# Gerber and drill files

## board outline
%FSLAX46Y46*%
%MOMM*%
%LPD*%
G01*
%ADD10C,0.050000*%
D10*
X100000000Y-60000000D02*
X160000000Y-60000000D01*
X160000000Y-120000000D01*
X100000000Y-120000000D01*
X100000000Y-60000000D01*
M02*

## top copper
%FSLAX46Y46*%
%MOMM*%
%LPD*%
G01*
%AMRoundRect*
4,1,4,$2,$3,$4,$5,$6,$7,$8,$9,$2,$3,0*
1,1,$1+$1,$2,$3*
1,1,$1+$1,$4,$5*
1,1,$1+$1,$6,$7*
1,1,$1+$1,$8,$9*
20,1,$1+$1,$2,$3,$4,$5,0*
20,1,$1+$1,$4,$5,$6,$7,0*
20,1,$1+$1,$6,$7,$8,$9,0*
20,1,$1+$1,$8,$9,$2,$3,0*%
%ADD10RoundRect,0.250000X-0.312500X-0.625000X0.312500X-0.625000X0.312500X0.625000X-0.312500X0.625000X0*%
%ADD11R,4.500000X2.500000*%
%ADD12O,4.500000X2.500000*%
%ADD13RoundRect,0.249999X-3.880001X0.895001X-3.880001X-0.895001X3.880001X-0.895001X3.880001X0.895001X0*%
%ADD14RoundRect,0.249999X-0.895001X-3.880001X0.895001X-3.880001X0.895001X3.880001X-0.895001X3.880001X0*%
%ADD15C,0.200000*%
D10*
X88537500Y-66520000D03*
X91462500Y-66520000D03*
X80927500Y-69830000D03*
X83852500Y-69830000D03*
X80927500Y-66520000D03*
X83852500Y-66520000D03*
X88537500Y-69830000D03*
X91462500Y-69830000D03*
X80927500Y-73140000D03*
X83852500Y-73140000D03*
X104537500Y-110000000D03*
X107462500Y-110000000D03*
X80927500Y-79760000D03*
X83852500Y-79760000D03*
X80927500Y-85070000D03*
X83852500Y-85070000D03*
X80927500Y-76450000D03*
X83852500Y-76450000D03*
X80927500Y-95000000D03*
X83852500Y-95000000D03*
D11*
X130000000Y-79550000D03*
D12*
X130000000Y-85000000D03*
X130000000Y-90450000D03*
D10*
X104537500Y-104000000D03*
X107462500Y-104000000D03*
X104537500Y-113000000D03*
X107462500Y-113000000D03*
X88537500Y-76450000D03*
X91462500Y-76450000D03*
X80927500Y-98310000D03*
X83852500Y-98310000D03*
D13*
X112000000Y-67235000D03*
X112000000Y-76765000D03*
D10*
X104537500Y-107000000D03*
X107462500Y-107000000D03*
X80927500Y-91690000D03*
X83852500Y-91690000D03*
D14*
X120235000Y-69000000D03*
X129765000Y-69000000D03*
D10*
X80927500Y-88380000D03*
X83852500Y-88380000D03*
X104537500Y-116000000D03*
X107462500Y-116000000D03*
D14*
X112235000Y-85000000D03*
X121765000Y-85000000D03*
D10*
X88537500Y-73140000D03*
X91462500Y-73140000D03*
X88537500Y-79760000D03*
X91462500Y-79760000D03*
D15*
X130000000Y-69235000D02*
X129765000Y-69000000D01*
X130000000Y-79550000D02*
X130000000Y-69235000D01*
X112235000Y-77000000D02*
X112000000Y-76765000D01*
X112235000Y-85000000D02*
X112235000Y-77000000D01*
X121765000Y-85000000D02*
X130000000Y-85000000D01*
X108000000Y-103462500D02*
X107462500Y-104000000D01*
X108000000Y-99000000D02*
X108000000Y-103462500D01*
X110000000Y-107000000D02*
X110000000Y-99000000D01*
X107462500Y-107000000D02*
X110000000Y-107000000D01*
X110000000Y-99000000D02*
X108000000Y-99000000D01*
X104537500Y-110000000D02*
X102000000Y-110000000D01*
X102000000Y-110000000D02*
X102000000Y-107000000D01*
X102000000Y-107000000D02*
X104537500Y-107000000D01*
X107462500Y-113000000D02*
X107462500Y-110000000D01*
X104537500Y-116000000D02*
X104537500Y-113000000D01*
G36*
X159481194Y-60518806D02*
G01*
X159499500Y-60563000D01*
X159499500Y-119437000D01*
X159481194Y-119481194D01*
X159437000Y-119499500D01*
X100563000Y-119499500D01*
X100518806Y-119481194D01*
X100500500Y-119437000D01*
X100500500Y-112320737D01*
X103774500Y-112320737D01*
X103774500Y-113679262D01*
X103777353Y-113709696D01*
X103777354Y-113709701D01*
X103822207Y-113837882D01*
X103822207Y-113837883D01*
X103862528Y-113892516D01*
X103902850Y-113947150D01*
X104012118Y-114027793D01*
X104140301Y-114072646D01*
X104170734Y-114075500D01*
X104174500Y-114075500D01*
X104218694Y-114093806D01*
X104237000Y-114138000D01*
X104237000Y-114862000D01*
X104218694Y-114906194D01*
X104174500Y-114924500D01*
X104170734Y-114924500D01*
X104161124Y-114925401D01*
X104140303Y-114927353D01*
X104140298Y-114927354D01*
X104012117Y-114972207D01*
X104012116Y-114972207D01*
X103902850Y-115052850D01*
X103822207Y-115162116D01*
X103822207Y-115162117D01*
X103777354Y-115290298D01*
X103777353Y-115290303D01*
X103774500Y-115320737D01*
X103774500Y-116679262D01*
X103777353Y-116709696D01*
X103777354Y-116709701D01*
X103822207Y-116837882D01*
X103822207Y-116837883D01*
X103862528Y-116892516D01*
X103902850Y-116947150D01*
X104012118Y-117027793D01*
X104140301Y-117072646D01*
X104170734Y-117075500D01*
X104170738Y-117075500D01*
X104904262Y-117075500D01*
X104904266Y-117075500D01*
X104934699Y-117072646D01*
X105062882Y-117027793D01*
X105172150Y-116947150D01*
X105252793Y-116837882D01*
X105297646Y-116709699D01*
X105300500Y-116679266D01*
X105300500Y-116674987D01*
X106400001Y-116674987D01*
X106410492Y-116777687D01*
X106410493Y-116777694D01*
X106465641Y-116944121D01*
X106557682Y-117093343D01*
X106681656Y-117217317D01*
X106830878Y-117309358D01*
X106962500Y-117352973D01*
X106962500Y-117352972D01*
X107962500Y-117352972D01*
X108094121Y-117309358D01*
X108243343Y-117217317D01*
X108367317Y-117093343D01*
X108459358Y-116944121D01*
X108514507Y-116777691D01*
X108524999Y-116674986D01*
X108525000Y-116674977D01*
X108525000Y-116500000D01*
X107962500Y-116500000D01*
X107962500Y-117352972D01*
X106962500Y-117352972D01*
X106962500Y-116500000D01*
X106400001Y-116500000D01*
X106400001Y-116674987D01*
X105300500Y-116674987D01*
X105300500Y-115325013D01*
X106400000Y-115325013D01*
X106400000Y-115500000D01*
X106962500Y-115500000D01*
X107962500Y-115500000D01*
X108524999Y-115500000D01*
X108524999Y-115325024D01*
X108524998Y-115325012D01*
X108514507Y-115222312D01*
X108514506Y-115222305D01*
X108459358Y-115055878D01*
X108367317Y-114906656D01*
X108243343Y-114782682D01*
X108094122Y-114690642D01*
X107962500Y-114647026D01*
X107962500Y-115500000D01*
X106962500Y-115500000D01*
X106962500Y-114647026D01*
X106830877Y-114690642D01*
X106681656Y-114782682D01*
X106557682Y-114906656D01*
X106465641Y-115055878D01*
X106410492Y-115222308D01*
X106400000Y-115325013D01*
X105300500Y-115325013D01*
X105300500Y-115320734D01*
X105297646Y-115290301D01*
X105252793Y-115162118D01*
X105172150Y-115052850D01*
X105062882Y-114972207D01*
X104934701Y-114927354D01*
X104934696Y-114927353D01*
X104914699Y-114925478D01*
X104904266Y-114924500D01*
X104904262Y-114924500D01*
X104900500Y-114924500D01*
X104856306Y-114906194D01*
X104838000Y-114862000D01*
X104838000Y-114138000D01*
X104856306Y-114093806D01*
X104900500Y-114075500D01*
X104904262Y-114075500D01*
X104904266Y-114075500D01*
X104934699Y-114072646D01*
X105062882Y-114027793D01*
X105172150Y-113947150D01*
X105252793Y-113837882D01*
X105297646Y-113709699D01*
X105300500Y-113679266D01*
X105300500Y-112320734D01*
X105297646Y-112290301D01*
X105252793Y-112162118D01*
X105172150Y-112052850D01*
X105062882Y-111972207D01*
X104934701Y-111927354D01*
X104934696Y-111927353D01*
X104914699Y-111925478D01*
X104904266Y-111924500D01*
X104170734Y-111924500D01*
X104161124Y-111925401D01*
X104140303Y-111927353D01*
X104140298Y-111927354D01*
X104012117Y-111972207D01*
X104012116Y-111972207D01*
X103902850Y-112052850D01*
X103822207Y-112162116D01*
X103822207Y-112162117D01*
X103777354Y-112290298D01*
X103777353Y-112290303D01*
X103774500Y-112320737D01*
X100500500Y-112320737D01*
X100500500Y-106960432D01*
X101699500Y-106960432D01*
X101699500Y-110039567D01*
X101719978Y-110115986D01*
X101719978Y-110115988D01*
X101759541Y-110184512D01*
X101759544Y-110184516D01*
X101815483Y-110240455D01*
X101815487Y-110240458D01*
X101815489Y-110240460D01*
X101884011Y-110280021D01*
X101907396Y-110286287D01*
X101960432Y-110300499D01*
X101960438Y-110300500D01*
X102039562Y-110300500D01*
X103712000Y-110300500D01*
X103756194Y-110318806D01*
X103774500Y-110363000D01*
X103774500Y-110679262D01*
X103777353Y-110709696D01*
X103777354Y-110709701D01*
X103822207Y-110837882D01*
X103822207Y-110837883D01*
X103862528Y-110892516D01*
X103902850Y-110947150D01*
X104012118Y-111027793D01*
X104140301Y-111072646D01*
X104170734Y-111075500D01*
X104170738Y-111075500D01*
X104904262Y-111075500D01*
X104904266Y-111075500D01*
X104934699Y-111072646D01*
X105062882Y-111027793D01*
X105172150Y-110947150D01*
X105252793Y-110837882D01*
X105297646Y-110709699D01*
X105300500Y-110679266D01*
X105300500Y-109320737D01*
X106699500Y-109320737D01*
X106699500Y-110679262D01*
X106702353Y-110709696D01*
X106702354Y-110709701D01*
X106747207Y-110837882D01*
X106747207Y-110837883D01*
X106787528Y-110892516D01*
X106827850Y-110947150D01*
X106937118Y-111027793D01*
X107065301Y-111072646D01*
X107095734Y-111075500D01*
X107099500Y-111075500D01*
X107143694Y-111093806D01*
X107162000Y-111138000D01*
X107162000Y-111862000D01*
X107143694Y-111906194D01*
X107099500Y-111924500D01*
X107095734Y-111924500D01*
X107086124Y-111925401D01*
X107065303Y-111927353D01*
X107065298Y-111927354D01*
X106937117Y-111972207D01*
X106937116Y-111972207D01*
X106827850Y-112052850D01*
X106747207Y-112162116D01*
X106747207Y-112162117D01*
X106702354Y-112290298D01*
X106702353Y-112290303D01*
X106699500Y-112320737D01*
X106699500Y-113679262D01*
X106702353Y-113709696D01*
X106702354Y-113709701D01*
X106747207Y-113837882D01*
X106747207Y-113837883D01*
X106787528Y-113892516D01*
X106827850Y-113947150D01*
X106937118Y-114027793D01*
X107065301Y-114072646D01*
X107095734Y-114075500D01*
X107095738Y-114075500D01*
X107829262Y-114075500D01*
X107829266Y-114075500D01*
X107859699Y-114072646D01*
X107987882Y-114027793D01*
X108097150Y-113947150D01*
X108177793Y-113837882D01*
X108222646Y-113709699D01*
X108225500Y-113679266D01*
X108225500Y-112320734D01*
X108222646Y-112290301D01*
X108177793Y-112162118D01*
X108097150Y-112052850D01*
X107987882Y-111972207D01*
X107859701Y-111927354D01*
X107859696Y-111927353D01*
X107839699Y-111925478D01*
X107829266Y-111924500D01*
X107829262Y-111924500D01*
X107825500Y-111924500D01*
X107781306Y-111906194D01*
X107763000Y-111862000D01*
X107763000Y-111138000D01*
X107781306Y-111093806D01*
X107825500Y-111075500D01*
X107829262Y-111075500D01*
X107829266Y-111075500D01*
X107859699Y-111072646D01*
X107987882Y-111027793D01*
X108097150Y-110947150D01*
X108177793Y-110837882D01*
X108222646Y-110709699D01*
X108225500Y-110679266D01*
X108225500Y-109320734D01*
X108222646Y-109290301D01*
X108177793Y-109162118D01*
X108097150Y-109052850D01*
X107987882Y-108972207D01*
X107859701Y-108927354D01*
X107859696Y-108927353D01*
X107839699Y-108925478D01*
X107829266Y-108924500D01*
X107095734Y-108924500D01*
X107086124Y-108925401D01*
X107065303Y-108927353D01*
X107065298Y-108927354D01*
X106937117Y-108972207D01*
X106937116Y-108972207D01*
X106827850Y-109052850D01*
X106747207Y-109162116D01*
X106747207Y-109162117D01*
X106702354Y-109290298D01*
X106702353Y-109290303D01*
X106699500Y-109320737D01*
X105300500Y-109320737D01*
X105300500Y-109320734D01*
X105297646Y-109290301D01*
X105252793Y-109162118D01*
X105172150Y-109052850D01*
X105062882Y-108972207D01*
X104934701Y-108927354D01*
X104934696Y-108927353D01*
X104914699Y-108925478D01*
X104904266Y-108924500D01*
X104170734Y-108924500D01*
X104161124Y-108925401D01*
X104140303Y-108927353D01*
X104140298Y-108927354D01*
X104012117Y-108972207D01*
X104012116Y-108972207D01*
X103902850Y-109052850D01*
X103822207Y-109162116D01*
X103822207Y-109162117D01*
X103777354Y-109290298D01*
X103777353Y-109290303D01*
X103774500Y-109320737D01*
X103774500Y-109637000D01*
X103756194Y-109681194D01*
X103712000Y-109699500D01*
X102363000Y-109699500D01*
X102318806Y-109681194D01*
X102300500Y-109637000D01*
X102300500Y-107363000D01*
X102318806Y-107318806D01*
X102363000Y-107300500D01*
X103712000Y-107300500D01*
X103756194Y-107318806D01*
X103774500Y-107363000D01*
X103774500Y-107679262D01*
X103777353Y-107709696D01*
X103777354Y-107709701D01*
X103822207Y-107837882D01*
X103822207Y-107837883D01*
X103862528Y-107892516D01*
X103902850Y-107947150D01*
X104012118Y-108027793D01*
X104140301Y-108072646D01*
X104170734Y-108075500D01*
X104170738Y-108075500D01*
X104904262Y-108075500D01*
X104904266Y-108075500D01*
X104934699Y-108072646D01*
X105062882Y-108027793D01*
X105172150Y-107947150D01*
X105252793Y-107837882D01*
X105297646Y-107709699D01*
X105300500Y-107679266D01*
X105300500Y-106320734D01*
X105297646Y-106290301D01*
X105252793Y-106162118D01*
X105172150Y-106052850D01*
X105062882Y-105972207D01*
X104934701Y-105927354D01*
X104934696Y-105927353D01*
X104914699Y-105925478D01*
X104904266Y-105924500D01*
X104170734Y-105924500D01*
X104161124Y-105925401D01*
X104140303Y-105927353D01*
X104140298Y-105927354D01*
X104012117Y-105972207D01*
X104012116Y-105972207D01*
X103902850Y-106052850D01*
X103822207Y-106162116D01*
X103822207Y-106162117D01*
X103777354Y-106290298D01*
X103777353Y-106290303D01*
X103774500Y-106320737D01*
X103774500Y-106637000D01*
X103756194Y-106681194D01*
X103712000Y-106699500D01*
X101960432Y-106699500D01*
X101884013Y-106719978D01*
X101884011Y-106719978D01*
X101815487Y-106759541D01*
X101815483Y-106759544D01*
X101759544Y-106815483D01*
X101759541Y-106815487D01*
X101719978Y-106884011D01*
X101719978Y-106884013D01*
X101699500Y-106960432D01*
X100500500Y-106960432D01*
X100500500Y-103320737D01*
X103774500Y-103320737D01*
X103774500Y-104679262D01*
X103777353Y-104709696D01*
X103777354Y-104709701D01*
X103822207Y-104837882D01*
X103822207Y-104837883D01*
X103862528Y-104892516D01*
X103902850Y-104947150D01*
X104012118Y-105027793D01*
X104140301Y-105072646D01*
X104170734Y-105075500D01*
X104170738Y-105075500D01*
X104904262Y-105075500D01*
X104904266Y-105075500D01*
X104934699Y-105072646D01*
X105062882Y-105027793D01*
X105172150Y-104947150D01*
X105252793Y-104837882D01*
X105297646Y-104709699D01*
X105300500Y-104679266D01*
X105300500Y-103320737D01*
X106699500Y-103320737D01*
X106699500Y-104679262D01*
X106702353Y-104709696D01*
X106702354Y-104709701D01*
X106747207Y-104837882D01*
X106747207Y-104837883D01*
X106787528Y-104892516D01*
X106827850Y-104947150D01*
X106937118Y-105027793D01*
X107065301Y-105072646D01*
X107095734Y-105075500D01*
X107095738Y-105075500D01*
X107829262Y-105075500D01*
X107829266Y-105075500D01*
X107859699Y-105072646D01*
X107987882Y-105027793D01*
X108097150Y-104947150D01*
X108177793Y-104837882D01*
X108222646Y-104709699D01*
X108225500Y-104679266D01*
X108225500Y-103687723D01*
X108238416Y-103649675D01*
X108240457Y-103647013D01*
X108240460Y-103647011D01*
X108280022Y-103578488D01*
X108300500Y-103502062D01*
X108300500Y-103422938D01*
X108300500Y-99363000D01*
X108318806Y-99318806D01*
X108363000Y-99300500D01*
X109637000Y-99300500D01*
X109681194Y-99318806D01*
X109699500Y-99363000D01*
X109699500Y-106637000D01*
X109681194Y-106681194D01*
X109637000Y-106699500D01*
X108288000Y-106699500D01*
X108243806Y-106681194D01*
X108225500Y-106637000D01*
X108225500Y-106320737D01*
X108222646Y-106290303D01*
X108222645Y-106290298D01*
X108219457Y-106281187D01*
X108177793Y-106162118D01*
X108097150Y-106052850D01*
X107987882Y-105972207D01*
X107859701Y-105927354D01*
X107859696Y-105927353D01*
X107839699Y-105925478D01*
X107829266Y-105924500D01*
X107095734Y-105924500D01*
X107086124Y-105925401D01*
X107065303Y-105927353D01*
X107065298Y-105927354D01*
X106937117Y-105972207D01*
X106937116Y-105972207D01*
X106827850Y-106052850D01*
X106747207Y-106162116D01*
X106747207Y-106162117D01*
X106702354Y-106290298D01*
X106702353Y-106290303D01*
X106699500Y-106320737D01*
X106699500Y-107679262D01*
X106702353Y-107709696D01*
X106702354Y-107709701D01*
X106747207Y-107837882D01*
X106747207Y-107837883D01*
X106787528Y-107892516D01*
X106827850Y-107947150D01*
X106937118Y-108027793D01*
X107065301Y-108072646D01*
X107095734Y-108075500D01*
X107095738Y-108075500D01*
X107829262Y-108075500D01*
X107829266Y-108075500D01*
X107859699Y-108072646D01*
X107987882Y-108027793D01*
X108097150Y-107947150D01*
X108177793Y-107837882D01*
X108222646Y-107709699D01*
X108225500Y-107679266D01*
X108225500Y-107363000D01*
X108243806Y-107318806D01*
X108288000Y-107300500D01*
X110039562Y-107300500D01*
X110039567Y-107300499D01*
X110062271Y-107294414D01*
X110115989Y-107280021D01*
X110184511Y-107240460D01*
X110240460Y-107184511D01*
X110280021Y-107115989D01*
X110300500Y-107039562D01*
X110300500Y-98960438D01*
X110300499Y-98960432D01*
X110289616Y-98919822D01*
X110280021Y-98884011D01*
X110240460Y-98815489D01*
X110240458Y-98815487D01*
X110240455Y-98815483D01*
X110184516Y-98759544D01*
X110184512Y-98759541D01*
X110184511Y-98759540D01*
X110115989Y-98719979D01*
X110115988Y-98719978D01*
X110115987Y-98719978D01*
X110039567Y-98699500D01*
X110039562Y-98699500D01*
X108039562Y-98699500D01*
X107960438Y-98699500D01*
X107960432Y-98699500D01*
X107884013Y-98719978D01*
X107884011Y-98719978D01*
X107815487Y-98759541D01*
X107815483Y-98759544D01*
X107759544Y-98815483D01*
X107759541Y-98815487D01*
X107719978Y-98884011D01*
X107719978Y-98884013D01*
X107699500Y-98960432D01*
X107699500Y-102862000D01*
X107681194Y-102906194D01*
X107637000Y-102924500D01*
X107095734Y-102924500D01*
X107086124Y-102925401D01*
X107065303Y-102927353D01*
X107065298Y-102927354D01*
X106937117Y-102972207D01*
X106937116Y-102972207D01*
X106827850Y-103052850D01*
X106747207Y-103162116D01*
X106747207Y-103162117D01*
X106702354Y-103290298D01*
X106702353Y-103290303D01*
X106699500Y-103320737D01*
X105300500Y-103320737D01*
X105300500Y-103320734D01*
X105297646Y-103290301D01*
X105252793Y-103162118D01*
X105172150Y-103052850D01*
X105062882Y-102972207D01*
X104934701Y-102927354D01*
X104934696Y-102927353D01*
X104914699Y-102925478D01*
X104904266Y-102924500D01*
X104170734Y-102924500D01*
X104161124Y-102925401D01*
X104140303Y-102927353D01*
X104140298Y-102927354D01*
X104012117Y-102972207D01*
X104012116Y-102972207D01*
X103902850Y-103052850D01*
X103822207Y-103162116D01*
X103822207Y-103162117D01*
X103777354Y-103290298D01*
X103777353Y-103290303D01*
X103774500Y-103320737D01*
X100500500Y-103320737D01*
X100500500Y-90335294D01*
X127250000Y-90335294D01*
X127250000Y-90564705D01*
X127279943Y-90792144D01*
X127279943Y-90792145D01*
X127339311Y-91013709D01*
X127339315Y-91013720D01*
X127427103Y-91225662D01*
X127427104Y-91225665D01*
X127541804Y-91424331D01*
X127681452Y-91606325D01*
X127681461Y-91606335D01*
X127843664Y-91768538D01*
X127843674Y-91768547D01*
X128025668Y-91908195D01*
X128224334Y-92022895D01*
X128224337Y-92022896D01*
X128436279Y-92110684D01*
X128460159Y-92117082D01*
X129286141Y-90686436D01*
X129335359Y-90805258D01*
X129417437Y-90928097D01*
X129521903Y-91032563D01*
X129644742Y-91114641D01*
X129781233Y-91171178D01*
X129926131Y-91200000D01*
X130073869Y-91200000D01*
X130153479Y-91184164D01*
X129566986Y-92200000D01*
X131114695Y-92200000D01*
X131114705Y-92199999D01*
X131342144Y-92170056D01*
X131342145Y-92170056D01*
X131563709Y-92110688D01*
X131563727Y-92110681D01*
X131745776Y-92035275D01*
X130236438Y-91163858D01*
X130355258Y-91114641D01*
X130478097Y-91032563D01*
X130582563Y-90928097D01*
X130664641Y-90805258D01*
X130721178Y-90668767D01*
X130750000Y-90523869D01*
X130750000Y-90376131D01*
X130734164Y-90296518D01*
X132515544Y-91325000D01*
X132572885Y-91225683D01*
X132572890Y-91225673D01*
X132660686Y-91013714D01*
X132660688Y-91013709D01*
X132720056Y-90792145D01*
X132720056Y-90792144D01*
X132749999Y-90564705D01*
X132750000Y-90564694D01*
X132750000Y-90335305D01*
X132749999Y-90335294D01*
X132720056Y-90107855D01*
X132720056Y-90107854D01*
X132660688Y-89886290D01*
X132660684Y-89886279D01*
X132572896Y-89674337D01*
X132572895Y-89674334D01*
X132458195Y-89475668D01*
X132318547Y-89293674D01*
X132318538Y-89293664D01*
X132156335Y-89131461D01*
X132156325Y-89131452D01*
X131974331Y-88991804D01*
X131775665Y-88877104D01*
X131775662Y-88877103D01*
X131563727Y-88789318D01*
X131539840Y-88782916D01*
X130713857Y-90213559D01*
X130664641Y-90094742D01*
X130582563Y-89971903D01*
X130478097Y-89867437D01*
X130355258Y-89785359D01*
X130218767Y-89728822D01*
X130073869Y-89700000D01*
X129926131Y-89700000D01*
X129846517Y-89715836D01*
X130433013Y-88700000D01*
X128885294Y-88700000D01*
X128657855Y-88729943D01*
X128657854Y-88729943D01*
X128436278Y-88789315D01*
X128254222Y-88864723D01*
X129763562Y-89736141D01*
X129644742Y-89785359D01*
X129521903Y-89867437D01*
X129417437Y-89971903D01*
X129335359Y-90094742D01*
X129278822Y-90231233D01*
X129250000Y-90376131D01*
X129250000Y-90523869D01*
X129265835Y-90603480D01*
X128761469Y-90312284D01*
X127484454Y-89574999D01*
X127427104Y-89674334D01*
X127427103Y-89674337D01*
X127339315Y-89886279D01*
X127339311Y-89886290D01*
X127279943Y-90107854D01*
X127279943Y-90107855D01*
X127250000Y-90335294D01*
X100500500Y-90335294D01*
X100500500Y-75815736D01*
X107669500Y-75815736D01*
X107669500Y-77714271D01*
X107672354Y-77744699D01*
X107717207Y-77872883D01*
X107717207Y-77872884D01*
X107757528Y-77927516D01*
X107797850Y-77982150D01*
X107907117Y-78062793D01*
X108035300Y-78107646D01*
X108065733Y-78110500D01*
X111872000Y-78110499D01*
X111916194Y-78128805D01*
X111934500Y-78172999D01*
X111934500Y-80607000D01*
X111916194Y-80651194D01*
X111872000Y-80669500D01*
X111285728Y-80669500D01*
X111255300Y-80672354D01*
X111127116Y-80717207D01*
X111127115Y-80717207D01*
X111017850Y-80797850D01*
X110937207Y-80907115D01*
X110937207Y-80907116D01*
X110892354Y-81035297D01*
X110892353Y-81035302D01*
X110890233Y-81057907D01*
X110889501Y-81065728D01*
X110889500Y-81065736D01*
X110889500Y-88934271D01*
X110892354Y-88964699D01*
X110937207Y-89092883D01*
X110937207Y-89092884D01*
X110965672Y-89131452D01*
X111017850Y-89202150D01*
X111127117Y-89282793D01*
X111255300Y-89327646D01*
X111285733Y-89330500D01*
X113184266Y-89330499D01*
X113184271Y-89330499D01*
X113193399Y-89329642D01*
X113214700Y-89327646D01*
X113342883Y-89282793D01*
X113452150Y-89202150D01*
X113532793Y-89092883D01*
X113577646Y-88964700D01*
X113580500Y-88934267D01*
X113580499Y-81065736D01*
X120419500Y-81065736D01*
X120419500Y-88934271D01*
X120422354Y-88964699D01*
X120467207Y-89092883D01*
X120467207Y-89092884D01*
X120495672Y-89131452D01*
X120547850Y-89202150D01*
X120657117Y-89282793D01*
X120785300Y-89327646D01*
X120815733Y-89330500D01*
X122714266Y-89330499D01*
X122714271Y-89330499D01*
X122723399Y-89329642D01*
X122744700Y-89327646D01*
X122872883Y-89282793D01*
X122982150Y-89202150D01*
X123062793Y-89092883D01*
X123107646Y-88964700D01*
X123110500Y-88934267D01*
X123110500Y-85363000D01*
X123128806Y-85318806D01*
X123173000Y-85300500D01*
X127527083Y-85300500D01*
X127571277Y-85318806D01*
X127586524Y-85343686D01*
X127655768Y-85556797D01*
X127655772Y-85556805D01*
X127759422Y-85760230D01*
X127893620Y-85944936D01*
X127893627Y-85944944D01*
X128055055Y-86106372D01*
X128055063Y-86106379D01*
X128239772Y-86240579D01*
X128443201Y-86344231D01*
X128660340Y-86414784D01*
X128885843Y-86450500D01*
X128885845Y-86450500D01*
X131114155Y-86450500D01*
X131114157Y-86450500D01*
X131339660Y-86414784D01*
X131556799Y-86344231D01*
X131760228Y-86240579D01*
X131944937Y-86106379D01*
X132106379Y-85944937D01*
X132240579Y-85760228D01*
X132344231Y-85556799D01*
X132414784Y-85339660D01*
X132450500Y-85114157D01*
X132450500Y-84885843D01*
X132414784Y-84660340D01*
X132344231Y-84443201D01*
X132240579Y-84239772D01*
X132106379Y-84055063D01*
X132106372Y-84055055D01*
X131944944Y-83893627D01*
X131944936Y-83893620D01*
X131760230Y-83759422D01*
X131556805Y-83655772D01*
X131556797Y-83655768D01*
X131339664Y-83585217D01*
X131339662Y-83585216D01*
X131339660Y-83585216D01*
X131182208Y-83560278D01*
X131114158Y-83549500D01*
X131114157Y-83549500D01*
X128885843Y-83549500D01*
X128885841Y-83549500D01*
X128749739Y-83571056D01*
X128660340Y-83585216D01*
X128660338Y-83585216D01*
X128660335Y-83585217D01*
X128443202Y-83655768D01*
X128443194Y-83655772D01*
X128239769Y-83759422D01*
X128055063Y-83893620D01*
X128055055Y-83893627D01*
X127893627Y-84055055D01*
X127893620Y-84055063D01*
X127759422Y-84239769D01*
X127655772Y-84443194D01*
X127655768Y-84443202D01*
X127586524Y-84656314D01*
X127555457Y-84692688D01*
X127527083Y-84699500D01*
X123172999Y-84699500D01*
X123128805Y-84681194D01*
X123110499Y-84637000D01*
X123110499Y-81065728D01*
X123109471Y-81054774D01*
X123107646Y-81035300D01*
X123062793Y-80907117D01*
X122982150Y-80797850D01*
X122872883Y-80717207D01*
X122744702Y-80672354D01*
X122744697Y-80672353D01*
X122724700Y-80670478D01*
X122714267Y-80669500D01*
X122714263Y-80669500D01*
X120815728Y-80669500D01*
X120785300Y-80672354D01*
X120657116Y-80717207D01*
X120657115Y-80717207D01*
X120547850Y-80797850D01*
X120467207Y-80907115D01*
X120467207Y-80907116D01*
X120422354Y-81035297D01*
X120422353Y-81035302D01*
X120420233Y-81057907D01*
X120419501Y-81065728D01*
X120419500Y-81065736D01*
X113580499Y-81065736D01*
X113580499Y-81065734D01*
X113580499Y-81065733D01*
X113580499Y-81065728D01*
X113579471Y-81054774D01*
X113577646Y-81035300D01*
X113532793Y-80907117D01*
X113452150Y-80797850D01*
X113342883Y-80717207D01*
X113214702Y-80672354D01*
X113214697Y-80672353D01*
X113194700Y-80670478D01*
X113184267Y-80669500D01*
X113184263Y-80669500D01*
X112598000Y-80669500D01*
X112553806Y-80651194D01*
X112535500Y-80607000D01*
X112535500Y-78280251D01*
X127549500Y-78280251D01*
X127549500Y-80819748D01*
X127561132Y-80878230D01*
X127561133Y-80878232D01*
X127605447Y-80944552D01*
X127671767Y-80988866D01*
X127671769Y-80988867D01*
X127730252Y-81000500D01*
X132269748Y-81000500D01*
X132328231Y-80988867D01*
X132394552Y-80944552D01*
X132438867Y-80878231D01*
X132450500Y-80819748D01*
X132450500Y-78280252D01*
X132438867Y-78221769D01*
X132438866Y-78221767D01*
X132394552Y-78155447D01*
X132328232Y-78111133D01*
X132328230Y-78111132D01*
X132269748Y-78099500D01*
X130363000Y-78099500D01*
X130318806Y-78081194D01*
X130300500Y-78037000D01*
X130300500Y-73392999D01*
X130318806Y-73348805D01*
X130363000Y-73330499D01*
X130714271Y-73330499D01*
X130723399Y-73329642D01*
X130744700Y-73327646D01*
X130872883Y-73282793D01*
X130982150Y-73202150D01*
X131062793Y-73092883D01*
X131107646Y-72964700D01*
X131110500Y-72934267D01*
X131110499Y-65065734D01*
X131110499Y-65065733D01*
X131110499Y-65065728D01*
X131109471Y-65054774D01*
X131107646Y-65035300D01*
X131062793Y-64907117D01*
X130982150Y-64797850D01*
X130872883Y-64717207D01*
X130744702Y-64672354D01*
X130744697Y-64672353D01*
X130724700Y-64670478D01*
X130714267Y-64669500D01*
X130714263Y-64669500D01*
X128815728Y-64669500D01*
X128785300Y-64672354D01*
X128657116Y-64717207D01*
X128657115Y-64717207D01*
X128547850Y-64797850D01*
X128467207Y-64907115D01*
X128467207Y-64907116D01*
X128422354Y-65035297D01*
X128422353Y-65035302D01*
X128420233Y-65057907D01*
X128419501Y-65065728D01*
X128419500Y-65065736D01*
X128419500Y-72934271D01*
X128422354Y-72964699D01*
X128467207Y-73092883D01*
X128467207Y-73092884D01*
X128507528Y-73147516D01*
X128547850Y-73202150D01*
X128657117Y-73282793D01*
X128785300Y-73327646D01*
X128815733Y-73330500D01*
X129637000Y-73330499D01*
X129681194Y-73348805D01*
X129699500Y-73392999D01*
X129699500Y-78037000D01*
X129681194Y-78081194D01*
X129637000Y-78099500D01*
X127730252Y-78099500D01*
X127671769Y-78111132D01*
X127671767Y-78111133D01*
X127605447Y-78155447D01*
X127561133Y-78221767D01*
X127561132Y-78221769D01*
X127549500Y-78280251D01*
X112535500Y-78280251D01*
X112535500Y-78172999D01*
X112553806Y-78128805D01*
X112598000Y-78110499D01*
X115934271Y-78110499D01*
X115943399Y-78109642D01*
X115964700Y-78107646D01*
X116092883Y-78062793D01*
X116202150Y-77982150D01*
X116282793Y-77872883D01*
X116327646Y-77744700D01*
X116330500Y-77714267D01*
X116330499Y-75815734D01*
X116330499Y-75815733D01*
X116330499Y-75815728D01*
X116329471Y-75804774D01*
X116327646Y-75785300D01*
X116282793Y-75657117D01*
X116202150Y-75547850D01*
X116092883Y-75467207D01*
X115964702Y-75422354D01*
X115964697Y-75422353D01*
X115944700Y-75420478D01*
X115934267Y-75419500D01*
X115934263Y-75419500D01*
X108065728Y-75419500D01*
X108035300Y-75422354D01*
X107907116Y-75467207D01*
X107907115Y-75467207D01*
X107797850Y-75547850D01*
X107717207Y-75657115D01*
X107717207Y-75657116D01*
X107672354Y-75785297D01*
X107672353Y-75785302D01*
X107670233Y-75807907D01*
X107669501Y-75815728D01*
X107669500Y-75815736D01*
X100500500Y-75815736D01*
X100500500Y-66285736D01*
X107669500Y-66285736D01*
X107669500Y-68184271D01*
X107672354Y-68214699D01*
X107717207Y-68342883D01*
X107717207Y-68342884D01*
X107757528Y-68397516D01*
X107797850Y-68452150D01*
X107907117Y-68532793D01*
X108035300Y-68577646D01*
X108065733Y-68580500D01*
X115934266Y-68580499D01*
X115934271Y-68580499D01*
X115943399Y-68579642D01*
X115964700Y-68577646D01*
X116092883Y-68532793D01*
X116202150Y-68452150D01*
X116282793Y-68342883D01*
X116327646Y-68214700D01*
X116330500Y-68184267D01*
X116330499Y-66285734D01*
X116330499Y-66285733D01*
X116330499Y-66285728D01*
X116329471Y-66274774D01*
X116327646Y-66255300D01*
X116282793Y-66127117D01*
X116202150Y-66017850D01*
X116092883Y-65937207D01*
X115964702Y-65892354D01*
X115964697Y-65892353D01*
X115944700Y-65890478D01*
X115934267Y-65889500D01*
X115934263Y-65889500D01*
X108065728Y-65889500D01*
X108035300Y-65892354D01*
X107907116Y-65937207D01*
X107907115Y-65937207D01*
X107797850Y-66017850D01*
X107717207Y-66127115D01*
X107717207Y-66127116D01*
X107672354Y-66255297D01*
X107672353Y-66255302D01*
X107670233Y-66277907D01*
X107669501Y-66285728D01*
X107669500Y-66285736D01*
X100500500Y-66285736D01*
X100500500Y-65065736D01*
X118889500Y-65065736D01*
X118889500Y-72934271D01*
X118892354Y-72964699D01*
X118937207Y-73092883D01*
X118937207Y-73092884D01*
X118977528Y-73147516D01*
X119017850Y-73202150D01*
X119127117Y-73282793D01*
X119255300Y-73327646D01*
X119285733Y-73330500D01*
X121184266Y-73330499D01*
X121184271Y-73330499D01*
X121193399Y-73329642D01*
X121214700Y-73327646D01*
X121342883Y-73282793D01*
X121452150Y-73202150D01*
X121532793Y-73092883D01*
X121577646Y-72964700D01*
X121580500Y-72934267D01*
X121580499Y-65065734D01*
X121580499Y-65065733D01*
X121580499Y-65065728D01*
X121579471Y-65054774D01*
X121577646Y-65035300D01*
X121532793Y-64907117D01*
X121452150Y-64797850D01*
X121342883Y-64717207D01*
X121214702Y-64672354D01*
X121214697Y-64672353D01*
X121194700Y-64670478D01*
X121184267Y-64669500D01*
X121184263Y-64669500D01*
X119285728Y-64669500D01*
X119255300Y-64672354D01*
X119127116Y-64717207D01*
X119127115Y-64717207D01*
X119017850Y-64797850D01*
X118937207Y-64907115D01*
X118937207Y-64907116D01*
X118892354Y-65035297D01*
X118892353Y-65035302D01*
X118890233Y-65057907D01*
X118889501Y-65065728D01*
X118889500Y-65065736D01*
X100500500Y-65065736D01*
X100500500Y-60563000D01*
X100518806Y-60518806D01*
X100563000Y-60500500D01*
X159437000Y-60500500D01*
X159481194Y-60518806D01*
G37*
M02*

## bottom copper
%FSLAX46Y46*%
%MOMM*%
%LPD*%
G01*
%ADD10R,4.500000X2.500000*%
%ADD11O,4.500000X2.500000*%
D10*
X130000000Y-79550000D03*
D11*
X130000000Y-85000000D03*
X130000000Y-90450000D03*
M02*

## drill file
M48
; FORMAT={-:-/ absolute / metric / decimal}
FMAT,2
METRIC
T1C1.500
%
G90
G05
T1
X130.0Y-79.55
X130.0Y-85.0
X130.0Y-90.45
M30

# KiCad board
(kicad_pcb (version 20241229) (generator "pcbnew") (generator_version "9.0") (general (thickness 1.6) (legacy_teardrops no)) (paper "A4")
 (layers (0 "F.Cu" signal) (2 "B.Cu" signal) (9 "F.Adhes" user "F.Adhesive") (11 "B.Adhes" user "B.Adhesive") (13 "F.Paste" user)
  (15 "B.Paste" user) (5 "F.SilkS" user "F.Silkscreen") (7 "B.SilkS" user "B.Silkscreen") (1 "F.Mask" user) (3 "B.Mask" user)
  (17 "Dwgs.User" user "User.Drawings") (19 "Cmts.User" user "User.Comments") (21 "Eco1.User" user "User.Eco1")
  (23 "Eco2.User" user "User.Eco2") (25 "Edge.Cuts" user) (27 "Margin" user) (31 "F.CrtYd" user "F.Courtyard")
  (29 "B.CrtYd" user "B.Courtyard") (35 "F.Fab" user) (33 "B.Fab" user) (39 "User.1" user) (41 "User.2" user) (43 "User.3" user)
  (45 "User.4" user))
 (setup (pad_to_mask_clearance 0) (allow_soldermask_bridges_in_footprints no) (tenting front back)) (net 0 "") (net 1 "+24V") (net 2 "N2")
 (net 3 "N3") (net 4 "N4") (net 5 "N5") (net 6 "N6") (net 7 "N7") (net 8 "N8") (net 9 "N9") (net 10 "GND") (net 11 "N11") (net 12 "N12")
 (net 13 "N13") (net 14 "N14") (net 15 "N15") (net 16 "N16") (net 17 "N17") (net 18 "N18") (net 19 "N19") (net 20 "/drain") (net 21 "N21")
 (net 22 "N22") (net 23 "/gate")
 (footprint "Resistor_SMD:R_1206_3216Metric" (layer "F.Cu") (at 90 66.52)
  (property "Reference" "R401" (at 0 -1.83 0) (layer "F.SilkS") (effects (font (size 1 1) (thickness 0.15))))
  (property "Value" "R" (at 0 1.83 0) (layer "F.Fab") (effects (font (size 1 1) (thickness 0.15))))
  (pad "1" smd roundrect (at -1.4625 0) (size 1.125 1.75) (layers "F.Cu" "F.Mask" "F.Paste") (roundrect_rratio 0.222222) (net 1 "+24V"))
  (pad "2" smd roundrect (at 1.4625 0) (size 1.125 1.75) (layers "F.Cu" "F.Mask" "F.Paste") (roundrect_rratio 0.222222) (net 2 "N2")))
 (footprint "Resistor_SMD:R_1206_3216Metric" (layer "F.Cu") (at 82.39 69.83)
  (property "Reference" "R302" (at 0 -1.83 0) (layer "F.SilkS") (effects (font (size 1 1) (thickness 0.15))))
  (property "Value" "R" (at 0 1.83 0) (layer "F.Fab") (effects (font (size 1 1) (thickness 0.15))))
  (pad "1" smd roundrect (at -1.4625 0) (size 1.125 1.75) (layers "F.Cu" "F.Mask" "F.Paste") (roundrect_rratio 0.222222) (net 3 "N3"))
  (pad "2" smd roundrect (at 1.4625 0) (size 1.125 1.75) (layers "F.Cu" "F.Mask" "F.Paste") (roundrect_rratio 0.222222) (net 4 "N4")))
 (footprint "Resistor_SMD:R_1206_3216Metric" (layer "F.Cu") (at 82.39 66.52)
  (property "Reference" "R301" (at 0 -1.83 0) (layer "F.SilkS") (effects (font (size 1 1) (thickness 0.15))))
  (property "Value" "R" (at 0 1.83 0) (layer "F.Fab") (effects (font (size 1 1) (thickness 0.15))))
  (pad "1" smd roundrect (at -1.4625 0) (size 1.125 1.75) (layers "F.Cu" "F.Mask" "F.Paste") (roundrect_rratio 0.222222) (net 1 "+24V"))
  (pad "2" smd roundrect (at 1.4625 0) (size 1.125 1.75) (layers "F.Cu" "F.Mask" "F.Paste") (roundrect_rratio 0.222222) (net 4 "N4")))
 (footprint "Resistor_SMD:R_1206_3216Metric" (layer "F.Cu") (at 90 69.83)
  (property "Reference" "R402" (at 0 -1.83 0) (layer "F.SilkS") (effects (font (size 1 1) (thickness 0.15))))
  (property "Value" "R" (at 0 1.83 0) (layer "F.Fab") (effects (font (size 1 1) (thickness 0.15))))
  (pad "1" smd roundrect (at -1.4625 0) (size 1.125 1.75) (layers "F.Cu" "F.Mask" "F.Paste") (roundrect_rratio 0.222222) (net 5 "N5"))
  (pad "2" smd roundrect (at 1.4625 0) (size 1.125 1.75) (layers "F.Cu" "F.Mask" "F.Paste") (roundrect_rratio 0.222222) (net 2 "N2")))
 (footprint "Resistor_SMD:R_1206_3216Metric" (layer "F.Cu") (at 82.39 73.14)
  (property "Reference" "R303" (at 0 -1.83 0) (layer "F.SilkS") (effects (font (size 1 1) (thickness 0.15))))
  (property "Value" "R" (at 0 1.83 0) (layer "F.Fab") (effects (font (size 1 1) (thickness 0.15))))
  (pad "1" smd roundrect (at -1.4625 0) (size 1.125 1.75) (layers "F.Cu" "F.Mask" "F.Paste") (roundrect_rratio 0.222222) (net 3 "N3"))
  (pad "2" smd roundrect (at 1.4625 0) (size 1.125 1.75) (layers "F.Cu" "F.Mask" "F.Paste") (roundrect_rratio 0.222222) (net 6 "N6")))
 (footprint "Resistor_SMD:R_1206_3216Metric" (layer "F.Cu") (at 106 110)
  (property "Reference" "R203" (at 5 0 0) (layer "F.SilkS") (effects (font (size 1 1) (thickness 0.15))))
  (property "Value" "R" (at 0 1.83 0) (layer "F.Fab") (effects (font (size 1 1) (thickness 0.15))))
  (pad "1" smd roundrect (at -1.4625 0) (size 1.125 1.75) (layers "F.Cu" "F.Mask" "F.Paste") (roundrect_rratio 0.222222) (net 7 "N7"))
  (pad "2" smd roundrect (at 1.4625 0) (size 1.125 1.75) (layers "F.Cu" "F.Mask" "F.Paste") (roundrect_rratio 0.222222) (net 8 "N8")))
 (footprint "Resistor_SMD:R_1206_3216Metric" (layer "F.Cu") (at 82.39 79.76)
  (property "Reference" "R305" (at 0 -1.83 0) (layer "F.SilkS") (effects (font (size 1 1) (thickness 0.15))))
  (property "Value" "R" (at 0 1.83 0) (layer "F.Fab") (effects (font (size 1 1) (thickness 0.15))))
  (pad "1" smd roundrect (at -1.4625 0) (size 1.125 1.75) (layers "F.Cu" "F.Mask" "F.Paste") (roundrect_rratio 0.222222) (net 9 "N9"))
  (pad "2" smd roundrect (at 1.4625 0) (size 1.125 1.75) (layers "F.Cu" "F.Mask" "F.Paste") (roundrect_rratio 0.222222) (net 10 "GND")))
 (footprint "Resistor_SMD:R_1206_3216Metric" (layer "F.Cu") (at 82.39 85.07)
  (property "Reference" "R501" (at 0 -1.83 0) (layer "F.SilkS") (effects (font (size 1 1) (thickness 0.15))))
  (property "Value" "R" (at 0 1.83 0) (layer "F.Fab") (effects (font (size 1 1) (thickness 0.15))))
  (pad "1" smd roundrect (at -1.4625 0) (size 1.125 1.75) (layers "F.Cu" "F.Mask" "F.Paste") (roundrect_rratio 0.222222) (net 1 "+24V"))
  (pad "2" smd roundrect (at 1.4625 0) (size 1.125 1.75) (layers "F.Cu" "F.Mask" "F.Paste") (roundrect_rratio 0.222222) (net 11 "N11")))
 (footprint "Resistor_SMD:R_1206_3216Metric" (layer "F.Cu") (at 82.39 76.45)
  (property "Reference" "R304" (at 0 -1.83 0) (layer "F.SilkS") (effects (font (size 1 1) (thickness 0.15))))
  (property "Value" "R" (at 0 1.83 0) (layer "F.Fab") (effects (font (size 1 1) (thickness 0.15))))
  (pad "1" smd roundrect (at -1.4625 0) (size 1.125 1.75) (layers "F.Cu" "F.Mask" "F.Paste") (roundrect_rratio 0.222222) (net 9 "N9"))
  (pad "2" smd roundrect (at 1.4625 0) (size 1.125 1.75) (layers "F.Cu" "F.Mask" "F.Paste") (roundrect_rratio 0.222222) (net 6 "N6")))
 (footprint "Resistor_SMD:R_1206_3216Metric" (layer "F.Cu") (at 82.39 95)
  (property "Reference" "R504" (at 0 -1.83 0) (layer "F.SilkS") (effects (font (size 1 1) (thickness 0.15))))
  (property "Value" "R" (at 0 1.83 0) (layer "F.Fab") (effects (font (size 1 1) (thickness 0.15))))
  (pad "1" smd roundrect (at -1.4625 0) (size 1.125 1.75) (layers "F.Cu" "F.Mask" "F.Paste") (roundrect_rratio 0.222222) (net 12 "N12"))
  (pad "2" smd roundrect (at 1.4625 0) (size 1.125 1.75) (layers "F.Cu" "F.Mask" "F.Paste") (roundrect_rratio 0.222222) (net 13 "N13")))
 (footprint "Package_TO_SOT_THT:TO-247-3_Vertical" (layer "F.Cu") (at 130 79.55 -90)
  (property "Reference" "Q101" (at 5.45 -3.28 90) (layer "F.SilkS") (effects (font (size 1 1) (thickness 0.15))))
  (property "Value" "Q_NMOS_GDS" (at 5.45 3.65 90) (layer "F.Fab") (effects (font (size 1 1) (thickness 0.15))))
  (pad "1" thru_hole rect (at 0 0 270) (size 2.5 4.5) (drill 1.5) (layers "*.Cu" "*.Mask") (remove_unused_layers no) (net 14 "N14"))
  (pad "2" thru_hole oval (at 5.45 0 270) (size 2.5 4.5) (drill 1.5) (layers "*.Cu" "*.Mask") (remove_unused_layers no) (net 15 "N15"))
  (pad "3" thru_hole oval (at 10.9 0 270) (size 2.5 4.5) (drill 1.5) (layers "*.Cu" "*.Mask") (remove_unused_layers no) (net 10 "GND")
   (thermal_bridge_angle 30)))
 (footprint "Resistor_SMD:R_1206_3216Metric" (layer "F.Cu") (at 106 104)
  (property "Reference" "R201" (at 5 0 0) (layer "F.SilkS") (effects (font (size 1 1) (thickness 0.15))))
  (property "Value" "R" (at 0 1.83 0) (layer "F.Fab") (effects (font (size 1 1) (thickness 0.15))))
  (pad "1" smd roundrect (at -1.4625 0) (size 1.125 1.75) (layers "F.Cu" "F.Mask" "F.Paste") (roundrect_rratio 0.222222) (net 1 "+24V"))
  (pad "2" smd roundrect (at 1.4625 0) (size 1.125 1.75) (layers "F.Cu" "F.Mask" "F.Paste") (roundrect_rratio 0.222222) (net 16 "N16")))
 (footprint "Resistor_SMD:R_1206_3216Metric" (layer "F.Cu") (at 106 113)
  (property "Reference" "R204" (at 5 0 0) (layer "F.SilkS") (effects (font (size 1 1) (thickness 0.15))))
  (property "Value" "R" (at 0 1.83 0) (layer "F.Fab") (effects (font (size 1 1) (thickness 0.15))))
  (pad "1" smd roundrect (at -1.4625 0) (size 1.125 1.75) (layers "F.Cu" "F.Mask" "F.Paste") (roundrect_rratio 0.222222) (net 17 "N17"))
  (pad "2" smd roundrect (at 1.4625 0) (size 1.125 1.75) (layers "F.Cu" "F.Mask" "F.Paste") (roundrect_rratio 0.222222) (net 8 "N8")))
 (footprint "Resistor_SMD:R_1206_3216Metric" (layer "F.Cu") (at 90 76.45)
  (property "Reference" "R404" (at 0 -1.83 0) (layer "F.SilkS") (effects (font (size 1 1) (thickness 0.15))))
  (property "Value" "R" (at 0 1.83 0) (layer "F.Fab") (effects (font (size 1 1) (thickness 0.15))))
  (pad "1" smd roundrect (at -1.4625 0) (size 1.125 1.75) (layers "F.Cu" "F.Mask" "F.Paste") (roundrect_rratio 0.222222) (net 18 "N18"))
  (pad "2" smd roundrect (at 1.4625 0) (size 1.125 1.75) (layers "F.Cu" "F.Mask" "F.Paste") (roundrect_rratio 0.222222) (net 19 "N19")))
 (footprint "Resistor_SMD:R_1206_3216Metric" (layer "F.Cu") (at 82.39 98.31)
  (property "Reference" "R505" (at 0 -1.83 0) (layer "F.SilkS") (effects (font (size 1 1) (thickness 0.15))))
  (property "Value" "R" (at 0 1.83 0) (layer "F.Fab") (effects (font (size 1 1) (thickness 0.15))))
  (pad "1" smd roundrect (at -1.4625 0) (size 1.125 1.75) (layers "F.Cu" "F.Mask" "F.Paste") (roundrect_rratio 0.222222) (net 12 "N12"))
  (pad "2" smd roundrect (at 1.4625 0) (size 1.125 1.75) (layers "F.Cu" "F.Mask" "F.Paste") (roundrect_rratio 0.222222) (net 10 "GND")))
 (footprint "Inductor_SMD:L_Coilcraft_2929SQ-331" (layer "F.Cu") (at 112 72 -90)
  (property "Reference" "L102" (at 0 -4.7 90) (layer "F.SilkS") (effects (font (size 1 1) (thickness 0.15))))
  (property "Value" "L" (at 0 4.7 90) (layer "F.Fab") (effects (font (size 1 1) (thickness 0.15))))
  (pad "1" smd roundrect (at -4.765 0 270) (size 2.29 8.26) (layers "F.Cu" "F.Mask" "F.Paste") (roundrect_rratio 0.10917) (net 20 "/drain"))
  (pad "2" smd roundrect (at 4.765 0 270) (size 2.29 8.26) (layers "F.Cu" "F.Mask" "F.Paste") (roundrect_rratio 0.10917) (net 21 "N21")))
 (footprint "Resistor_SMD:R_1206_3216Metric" (layer "F.Cu") (at 106 107)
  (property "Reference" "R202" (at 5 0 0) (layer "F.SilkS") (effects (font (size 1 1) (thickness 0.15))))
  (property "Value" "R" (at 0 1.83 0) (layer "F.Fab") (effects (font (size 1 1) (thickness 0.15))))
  (pad "1" smd roundrect (at -1.4625 0) (size 1.125 1.75) (layers "F.Cu" "F.Mask" "F.Paste") (roundrect_rratio 0.222222) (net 7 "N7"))
  (pad "2" smd roundrect (at 1.4625 0) (size 1.125 1.75) (layers "F.Cu" "F.Mask" "F.Paste") (roundrect_rratio 0.222222) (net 16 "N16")))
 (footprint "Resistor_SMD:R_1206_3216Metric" (layer "F.Cu") (at 82.39 91.69)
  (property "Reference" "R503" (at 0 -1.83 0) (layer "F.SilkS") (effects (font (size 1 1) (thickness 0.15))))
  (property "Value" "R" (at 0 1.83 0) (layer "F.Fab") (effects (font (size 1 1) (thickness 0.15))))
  (pad "1" smd roundrect (at -1.4625 0) (size 1.125 1.75) (layers "F.Cu" "F.Mask" "F.Paste") (roundrect_rratio 0.222222) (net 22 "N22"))
  (pad "2" smd roundrect (at 1.4625 0) (size 1.125 1.75) (layers "F.Cu" "F.Mask" "F.Paste") (roundrect_rratio 0.222222) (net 13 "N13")))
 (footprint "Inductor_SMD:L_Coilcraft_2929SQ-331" (layer "F.Cu") (at 125 69)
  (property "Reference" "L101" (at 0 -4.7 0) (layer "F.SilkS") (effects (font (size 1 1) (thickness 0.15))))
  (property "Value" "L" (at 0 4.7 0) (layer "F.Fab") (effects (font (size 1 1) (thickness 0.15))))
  (pad "1" smd roundrect (at -4.765 0) (size 2.29 8.26) (layers "F.Cu" "F.Mask" "F.Paste") (roundrect_rratio 0.10917) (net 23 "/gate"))
  (pad "2" smd roundrect (at 4.765 0) (size 2.29 8.26) (layers "F.Cu" "F.Mask" "F.Paste") (roundrect_rratio 0.10917) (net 14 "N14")))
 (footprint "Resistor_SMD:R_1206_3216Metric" (layer "F.Cu") (at 82.39 88.38)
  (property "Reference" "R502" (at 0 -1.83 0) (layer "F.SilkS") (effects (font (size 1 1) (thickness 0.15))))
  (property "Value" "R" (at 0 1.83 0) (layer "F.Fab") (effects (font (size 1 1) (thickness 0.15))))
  (pad "1" smd roundrect (at -1.4625 0) (size 1.125 1.75) (layers "F.Cu" "F.Mask" "F.Paste") (roundrect_rratio 0.222222) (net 22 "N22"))
  (pad "2" smd roundrect (at 1.4625 0) (size 1.125 1.75) (layers "F.Cu" "F.Mask" "F.Paste") (roundrect_rratio 0.222222) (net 11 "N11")))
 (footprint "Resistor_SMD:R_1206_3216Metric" (layer "F.Cu") (at 106 116)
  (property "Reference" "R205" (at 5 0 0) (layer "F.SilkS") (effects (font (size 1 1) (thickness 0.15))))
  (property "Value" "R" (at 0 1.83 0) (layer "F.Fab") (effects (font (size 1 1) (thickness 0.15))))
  (pad "1" smd roundrect (at -1.4625 0) (size 1.125 1.75) (layers "F.Cu" "F.Mask" "F.Paste") (roundrect_rratio 0.222222) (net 17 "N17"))
  (pad "2" smd roundrect (at 1.4625 0) (size 1.125 1.75) (layers "F.Cu" "F.Mask" "F.Paste") (roundrect_rratio 0.222222) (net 10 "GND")))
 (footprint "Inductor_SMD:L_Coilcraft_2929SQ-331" (layer "F.Cu") (at 117 85)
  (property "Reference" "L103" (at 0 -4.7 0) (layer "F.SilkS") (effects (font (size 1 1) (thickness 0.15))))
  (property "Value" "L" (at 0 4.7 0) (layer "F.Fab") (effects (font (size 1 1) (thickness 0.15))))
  (pad "1" smd roundrect (at -4.765 0) (size 2.29 8.26) (layers "F.Cu" "F.Mask" "F.Paste") (roundrect_rratio 0.10917) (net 21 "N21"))
  (pad "2" smd roundrect (at 4.765 0) (size 2.29 8.26) (layers "F.Cu" "F.Mask" "F.Paste") (roundrect_rratio 0.10917) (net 15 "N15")))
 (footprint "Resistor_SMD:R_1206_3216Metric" (layer "F.Cu") (at 90 73.14)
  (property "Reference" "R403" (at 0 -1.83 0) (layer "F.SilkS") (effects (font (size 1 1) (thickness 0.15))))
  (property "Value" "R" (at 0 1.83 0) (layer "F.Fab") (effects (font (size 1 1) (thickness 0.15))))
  (pad "1" smd roundrect (at -1.4625 0) (size 1.125 1.75) (layers "F.Cu" "F.Mask" "F.Paste") (roundrect_rratio 0.222222) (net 5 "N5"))
  (pad "2" smd roundrect (at 1.4625 0) (size 1.125 1.75) (layers "F.Cu" "F.Mask" "F.Paste") (roundrect_rratio 0.222222) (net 19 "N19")))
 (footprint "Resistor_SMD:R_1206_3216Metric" (layer "F.Cu") (at 90 79.76)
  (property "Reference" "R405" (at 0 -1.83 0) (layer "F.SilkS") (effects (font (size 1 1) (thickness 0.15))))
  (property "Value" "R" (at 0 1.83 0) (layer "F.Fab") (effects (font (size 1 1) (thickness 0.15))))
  (pad "1" smd roundrect (at -1.4625 0) (size 1.125 1.75) (layers "F.Cu" "F.Mask" "F.Paste") (roundrect_rratio 0.222222) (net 18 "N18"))
  (pad "2" smd roundrect (at 1.4625 0) (size 1.125 1.75) (layers "F.Cu" "F.Mask" "F.Paste") (roundrect_rratio 0.222222) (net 10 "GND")))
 (gr_rect (start 100 60) (end 160 120) (stroke (width 0.05) (type default)) (fill no) (layer "Edge.Cuts"))
 (segment (start 130 69.235) (end 129.765 69) (width 0.2) (layer "F.Cu") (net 14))
 (segment (start 130 79.55) (end 130 69.235) (width 0.2) (layer "F.Cu") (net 14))
 (segment (start 112.235 77) (end 112 76.765) (width 0.2) (layer "F.Cu") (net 21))
 (segment (start 112.235 85) (end 112.235 77) (width 0.2) (layer "F.Cu") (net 21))
 (segment (start 121.765 85) (end 130 85) (width 0.2) (layer "F.Cu") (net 15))
 (segment (start 108 103.4625) (end 107.4625 104) (width 0.2) (layer "F.Cu") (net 16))
 (segment (start 108 99) (end 108 103.4625) (width 0.2) (layer "F.Cu") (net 16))
 (segment (start 110 107) (end 110 99) (width 0.2) (layer "F.Cu") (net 16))
 (segment (start 107.4625 107) (end 110 107) (width 0.2) (layer "F.Cu") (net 16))
 (segment (start 110 99) (end 108 99) (width 0.2) (layer "F.Cu") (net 16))
 (segment (start 104.5375 110) (end 102 110) (width 0.2) (layer "F.Cu") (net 7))
 (segment (start 102 110) (end 102 107) (width 0.2) (layer "F.Cu") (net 7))
 (segment (start 102 107) (end 104.5375 107) (width 0.2) (layer "F.Cu") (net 7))
 (segment (start 107.4625 113) (end 107.4625 110) (width 0.2) (layer "F.Cu") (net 8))
 (segment (start 104.5375 116) (end 104.5375 113) (width 0.2) (layer "F.Cu") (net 17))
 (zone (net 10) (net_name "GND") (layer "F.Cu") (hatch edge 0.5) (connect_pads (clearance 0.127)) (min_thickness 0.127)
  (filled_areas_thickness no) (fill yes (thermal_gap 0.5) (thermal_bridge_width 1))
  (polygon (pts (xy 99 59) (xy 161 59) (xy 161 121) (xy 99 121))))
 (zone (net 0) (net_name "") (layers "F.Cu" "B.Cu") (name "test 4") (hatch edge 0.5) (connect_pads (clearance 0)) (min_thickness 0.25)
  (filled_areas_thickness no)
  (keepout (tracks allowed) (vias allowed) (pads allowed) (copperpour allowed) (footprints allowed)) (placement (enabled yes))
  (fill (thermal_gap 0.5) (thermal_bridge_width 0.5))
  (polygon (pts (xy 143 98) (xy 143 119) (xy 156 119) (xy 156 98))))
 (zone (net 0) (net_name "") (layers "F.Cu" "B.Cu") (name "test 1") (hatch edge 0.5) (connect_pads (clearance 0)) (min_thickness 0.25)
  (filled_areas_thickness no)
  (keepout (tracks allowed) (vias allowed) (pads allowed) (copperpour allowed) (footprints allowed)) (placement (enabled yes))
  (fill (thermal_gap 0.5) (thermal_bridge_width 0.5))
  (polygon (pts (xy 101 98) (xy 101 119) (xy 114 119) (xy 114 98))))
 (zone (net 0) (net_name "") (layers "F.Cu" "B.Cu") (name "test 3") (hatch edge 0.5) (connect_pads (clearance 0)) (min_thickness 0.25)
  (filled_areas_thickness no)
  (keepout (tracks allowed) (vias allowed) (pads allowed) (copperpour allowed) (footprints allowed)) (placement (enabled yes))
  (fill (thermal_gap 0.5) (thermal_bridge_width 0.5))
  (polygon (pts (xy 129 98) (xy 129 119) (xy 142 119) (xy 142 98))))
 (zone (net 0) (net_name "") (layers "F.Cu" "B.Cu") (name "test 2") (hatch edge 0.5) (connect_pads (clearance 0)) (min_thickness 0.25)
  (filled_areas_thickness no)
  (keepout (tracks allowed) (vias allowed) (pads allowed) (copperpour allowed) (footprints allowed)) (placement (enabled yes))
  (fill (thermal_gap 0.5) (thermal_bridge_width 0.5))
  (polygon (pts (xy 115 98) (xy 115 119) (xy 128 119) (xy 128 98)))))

